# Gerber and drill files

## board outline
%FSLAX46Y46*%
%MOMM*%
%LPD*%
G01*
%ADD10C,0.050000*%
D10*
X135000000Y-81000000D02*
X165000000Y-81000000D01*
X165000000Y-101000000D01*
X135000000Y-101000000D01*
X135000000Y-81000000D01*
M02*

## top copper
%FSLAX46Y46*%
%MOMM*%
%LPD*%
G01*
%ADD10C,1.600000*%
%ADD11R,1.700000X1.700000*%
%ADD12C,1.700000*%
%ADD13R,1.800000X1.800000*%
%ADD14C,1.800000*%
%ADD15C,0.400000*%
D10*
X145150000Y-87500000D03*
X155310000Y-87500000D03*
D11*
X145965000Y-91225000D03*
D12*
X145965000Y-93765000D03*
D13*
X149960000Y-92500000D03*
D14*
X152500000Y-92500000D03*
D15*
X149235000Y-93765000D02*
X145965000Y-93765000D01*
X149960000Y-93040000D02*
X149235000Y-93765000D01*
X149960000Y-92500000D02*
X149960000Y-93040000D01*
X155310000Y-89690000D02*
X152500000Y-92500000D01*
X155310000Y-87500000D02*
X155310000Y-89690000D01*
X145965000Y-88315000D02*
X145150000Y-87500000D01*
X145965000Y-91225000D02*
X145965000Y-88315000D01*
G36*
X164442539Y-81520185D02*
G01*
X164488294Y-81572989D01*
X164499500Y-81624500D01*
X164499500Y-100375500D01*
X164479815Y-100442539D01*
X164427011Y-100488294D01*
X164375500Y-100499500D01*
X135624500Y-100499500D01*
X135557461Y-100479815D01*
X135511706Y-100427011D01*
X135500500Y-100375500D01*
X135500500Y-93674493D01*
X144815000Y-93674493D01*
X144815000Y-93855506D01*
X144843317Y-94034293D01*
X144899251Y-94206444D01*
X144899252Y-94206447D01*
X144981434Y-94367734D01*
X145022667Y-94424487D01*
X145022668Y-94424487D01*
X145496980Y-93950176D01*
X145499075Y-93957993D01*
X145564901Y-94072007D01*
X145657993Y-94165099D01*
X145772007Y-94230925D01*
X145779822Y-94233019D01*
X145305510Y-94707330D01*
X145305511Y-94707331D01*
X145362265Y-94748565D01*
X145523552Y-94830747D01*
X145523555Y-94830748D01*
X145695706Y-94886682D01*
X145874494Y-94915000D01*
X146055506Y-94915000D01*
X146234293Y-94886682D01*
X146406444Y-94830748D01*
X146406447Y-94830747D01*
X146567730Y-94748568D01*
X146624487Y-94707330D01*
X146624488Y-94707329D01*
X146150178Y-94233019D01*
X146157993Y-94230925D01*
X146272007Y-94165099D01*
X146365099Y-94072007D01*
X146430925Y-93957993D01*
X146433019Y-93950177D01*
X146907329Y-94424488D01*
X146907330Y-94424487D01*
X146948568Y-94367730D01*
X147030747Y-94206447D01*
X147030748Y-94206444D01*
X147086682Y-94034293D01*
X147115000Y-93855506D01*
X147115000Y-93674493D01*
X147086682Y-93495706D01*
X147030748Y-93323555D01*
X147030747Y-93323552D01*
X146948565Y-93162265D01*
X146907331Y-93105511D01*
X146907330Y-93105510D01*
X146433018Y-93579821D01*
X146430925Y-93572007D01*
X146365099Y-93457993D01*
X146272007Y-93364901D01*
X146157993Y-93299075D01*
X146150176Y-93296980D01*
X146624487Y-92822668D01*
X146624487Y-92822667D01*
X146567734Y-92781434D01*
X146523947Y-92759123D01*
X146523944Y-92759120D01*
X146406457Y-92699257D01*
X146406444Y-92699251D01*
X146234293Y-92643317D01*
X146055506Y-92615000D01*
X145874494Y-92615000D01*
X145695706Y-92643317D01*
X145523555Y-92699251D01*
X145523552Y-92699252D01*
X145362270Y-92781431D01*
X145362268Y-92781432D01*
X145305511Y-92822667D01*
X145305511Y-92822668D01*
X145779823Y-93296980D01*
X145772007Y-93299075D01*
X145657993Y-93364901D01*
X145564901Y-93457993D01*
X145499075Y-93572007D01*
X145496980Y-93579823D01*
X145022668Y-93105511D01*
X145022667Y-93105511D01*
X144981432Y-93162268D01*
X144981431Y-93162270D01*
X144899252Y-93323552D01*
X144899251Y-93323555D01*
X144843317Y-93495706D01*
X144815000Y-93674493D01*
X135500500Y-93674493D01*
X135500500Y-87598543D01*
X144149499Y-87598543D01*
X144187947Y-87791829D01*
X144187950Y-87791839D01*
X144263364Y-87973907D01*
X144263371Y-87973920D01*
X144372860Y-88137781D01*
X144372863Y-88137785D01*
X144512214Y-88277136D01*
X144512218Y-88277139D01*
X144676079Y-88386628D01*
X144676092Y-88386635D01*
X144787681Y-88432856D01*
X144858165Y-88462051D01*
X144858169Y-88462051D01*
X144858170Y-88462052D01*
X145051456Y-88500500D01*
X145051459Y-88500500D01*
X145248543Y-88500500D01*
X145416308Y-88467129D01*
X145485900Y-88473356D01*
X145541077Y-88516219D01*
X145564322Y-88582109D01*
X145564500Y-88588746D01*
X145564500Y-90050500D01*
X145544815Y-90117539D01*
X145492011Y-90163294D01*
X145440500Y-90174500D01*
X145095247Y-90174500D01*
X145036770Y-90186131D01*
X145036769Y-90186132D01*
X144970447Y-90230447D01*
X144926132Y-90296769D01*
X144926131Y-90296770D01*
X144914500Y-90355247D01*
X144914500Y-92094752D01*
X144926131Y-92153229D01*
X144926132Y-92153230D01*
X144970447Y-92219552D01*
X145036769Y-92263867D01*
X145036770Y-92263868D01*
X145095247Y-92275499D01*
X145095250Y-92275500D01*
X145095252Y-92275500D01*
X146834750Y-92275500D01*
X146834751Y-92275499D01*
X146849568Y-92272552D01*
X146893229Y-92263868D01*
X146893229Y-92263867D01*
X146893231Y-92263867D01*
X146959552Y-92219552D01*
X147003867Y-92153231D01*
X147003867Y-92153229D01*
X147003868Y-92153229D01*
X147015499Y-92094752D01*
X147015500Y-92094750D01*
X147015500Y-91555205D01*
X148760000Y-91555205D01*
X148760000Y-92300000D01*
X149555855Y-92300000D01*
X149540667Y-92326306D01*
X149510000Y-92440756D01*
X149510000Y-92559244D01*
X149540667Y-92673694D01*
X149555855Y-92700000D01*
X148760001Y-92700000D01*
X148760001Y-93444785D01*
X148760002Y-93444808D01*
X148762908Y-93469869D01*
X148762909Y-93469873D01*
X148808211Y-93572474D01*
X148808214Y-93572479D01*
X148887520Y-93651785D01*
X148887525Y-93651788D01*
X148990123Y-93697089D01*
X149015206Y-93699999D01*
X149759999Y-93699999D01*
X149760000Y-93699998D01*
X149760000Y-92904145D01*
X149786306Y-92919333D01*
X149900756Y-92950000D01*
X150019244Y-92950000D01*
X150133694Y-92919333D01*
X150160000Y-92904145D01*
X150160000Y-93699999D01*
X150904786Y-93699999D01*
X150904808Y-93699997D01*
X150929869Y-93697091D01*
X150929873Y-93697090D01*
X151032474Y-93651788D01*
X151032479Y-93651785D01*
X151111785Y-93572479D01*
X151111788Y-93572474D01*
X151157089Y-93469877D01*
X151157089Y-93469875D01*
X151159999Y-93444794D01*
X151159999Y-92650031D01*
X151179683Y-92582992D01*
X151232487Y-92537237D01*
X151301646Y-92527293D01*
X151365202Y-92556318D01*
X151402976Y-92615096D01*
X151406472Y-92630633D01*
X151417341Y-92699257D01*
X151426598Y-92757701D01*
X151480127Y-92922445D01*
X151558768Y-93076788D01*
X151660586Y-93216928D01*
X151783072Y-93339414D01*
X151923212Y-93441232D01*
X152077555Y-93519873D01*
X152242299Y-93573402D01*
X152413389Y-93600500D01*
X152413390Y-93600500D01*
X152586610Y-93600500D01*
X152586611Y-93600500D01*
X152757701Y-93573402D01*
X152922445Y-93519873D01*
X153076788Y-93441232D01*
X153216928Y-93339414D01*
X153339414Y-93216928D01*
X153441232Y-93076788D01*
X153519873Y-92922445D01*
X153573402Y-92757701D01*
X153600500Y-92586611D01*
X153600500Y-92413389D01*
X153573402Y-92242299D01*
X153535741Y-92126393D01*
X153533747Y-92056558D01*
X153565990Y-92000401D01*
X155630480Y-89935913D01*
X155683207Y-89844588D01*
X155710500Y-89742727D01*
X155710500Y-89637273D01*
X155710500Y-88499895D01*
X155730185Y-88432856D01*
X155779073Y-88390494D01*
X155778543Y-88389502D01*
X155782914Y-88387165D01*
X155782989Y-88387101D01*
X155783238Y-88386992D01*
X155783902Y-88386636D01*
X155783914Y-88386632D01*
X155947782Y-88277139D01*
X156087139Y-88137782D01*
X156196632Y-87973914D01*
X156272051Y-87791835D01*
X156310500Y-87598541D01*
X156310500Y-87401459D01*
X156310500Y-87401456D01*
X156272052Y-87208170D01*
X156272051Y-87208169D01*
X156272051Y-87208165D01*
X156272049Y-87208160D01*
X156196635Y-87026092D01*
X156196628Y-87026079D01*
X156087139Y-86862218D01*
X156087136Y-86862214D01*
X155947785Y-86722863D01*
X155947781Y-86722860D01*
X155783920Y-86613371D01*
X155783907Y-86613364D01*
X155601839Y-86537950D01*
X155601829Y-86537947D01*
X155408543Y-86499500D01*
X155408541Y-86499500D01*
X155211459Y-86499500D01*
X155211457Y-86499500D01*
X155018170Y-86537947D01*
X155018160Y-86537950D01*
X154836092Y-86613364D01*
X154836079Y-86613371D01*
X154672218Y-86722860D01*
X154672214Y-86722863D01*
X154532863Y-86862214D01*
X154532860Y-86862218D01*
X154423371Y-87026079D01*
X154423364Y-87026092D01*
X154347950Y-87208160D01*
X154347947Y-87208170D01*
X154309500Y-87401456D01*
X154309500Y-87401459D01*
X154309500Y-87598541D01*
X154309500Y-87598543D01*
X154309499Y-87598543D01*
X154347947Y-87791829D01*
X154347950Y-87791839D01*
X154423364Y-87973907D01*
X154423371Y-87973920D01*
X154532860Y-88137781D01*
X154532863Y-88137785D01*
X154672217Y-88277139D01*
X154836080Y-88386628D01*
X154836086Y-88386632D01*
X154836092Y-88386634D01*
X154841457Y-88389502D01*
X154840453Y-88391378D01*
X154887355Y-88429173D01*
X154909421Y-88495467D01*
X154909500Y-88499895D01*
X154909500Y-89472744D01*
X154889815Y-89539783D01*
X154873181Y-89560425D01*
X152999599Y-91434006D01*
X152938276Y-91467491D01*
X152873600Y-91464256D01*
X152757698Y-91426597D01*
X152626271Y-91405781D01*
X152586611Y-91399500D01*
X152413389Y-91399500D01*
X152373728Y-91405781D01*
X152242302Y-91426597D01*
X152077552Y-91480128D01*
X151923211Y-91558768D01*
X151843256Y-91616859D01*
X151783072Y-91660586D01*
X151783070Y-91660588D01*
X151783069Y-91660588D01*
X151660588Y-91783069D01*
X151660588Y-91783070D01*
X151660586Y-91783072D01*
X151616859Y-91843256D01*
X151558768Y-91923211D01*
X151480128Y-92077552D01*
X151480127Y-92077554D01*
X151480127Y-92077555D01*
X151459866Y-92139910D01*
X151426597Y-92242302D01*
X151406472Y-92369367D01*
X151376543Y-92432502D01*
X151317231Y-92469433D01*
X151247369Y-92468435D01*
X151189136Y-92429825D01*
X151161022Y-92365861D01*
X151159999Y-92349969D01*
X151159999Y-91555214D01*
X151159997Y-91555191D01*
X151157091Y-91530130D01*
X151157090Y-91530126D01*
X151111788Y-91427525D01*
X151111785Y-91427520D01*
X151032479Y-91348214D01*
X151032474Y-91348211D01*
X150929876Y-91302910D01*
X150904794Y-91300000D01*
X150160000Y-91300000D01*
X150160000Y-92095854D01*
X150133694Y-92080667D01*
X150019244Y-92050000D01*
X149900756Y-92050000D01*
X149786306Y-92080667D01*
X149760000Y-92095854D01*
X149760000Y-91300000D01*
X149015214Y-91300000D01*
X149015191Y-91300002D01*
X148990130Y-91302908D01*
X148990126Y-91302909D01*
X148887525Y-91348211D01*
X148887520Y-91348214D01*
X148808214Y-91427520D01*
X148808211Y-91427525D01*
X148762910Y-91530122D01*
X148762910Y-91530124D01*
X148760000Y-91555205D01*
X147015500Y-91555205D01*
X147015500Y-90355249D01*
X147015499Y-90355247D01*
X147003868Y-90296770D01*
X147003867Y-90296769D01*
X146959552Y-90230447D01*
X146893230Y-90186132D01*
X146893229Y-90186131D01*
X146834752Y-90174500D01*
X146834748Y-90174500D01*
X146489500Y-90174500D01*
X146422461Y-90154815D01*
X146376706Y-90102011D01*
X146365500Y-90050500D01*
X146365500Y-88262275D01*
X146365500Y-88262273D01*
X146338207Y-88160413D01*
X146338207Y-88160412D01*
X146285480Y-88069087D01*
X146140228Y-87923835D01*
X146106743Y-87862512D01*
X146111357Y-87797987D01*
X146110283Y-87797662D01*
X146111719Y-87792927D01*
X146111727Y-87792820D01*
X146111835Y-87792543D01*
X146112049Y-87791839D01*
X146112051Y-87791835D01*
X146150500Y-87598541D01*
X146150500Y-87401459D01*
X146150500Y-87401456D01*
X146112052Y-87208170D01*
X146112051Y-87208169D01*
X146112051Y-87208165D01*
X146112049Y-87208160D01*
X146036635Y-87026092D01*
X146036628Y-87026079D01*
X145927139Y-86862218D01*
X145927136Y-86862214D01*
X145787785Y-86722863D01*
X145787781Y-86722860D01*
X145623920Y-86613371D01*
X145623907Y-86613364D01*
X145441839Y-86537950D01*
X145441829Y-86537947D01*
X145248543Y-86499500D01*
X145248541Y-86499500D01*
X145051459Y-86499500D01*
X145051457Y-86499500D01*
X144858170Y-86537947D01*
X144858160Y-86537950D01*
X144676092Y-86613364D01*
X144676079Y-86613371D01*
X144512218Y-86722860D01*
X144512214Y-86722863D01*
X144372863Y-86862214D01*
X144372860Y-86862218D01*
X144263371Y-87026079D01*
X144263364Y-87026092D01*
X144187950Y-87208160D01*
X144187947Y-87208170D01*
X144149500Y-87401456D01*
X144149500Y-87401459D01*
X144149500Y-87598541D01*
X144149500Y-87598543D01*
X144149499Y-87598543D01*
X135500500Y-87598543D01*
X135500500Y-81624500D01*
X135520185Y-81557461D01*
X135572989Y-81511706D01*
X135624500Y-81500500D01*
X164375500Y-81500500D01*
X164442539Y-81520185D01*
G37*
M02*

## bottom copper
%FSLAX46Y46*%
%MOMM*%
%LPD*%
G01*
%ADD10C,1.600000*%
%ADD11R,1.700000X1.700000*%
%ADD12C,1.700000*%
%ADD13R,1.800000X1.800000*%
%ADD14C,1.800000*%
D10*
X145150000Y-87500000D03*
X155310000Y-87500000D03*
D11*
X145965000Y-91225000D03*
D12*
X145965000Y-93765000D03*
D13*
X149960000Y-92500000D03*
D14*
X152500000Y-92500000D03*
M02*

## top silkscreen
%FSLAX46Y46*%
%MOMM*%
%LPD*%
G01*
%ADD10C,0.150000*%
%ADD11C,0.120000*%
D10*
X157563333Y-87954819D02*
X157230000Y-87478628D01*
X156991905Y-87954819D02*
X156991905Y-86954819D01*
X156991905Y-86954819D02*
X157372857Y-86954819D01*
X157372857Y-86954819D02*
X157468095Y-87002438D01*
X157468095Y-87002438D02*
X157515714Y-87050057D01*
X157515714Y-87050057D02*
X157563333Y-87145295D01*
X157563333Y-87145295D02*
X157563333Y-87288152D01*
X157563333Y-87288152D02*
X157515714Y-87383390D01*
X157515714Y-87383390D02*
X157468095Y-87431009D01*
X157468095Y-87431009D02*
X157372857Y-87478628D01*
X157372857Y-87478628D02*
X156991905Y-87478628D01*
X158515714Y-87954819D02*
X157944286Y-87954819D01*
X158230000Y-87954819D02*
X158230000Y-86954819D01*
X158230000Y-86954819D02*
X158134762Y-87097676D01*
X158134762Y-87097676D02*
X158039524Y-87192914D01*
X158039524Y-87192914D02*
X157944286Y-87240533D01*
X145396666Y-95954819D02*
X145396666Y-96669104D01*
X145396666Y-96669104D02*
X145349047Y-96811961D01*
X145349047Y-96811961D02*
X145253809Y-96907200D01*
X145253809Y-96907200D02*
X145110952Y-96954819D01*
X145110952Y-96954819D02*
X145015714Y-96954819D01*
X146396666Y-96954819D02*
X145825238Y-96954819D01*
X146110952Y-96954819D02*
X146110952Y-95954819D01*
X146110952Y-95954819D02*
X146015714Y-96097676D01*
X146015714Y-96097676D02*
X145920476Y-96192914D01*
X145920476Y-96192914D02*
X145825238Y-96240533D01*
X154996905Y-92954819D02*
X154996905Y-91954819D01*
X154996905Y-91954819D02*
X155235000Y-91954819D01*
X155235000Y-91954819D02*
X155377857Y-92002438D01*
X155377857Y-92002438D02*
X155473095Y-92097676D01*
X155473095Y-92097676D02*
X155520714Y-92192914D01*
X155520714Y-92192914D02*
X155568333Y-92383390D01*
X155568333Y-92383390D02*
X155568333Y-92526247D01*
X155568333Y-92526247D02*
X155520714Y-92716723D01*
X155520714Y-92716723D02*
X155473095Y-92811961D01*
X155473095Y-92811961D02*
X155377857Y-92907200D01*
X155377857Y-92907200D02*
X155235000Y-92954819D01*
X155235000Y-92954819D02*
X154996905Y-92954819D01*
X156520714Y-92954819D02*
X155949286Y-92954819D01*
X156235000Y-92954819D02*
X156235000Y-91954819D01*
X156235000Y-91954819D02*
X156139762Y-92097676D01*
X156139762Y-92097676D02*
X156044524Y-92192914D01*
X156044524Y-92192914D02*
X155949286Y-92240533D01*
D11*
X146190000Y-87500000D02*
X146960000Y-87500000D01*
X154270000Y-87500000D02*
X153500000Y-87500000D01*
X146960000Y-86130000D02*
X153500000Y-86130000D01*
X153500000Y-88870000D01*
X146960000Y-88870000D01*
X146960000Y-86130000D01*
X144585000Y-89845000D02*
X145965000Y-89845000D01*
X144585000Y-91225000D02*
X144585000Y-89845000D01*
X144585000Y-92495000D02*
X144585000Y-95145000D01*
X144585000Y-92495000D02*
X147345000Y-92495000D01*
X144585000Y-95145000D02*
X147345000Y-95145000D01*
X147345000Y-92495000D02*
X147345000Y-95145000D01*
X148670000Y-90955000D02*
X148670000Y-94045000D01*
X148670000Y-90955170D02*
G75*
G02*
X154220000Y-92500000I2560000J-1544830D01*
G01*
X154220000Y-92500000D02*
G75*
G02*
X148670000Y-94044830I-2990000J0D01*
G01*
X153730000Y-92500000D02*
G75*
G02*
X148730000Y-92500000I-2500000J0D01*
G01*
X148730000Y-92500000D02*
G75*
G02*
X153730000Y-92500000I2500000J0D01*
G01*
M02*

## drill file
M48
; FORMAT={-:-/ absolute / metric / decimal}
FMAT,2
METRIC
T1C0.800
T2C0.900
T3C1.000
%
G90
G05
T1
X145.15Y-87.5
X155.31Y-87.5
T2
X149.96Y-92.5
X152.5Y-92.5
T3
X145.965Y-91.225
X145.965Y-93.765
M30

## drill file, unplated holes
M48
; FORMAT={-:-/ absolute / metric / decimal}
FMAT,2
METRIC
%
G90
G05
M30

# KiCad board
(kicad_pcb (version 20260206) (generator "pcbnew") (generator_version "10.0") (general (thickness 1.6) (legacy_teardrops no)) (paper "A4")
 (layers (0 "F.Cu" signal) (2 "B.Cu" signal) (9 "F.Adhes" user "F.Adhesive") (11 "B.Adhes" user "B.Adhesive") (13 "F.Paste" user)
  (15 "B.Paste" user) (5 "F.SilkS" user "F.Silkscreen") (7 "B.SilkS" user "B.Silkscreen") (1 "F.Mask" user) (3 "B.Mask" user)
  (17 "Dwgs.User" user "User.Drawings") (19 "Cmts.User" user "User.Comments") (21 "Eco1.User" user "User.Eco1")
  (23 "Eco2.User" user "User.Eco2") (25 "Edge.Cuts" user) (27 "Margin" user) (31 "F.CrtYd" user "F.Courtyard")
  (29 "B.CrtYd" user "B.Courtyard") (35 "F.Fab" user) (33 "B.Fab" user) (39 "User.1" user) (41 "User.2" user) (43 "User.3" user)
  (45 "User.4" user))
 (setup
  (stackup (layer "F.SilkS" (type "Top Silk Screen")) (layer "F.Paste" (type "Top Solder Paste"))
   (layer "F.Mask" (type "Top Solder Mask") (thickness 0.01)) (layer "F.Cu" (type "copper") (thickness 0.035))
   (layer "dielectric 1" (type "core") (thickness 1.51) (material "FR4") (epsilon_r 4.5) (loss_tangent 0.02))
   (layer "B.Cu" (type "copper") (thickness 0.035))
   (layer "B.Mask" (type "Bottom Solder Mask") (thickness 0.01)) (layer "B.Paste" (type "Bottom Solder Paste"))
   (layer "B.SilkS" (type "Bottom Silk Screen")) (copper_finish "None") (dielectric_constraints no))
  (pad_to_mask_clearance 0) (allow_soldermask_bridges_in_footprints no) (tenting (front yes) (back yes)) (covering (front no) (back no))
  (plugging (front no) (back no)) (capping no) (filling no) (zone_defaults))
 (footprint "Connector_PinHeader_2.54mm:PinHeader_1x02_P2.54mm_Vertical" (layer "F.Cu") (at 145.965 91.225)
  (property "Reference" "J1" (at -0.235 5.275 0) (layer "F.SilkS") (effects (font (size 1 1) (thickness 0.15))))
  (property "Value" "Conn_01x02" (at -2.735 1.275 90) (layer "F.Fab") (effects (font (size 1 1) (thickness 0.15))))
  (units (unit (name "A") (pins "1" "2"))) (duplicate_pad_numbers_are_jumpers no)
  (fp_line (start -1.38 -1.38) (end 0 -1.38) (stroke (width 0.12) (type solid)) (layer "F.SilkS"))
  (fp_line (start -1.38 0) (end -1.38 -1.38) (stroke (width 0.12) (type solid)) (layer "F.SilkS"))
  (fp_line (start -1.38 1.27) (end -1.38 3.92) (stroke (width 0.12) (type solid)) (layer "F.SilkS"))
  (fp_line (start -1.38 1.27) (end 1.38 1.27) (stroke (width 0.12) (type solid)) (layer "F.SilkS"))
  (fp_line (start -1.38 3.92) (end 1.38 3.92) (stroke (width 0.12) (type solid)) (layer "F.SilkS"))
  (fp_line (start 1.38 1.27) (end 1.38 3.92) (stroke (width 0.12) (type solid)) (layer "F.SilkS"))
  (pad "1" thru_hole rect (at 0 0) (size 1.7 1.7) (drill 1) (layers "*.Cu" "*.Mask") (remove_unused_layers no) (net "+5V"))
  (pad "2" thru_hole circle (at 0 2.54) (size 1.7 1.7) (drill 1) (layers "*.Cu" "*.Mask") (remove_unused_layers no) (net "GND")))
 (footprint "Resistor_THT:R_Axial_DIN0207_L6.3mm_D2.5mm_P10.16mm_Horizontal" (layer "F.Cu") (at 145.15 87.5)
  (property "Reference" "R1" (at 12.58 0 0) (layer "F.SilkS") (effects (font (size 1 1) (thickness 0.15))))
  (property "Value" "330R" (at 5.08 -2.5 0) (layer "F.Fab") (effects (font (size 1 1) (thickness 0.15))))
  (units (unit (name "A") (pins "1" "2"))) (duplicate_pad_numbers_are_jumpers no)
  (fp_line (start 1.04 0) (end 1.81 0) (stroke (width 0.12) (type solid)) (layer "F.SilkS"))
  (fp_line (start 9.12 0) (end 8.35 0) (stroke (width 0.12) (type solid)) (layer "F.SilkS"))
  (fp_rect (start 1.81 -1.37) (end 8.35 1.37) (stroke (width 0.12) (type solid)) (fill no) (layer "F.SilkS"))
  (pad "1" thru_hole circle (at 0 0) (size 1.6 1.6) (drill 0.8) (layers "*.Cu" "*.Mask") (remove_unused_layers no) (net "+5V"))
  (pad "2" thru_hole circle (at 10.16 0) (size 1.6 1.6) (drill 0.8) (layers "*.Cu" "*.Mask") (remove_unused_layers no) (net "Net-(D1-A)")))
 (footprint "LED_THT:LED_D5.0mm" (layer "F.Cu") (at 149.96 92.5)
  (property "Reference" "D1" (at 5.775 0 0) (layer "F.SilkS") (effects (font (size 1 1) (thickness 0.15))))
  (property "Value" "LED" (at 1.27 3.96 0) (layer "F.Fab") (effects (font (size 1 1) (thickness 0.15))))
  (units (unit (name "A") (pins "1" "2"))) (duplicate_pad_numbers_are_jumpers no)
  (fp_line (start -1.29 -1.545) (end -1.29 1.545) (stroke (width 0.12) (type solid)) (layer "F.SilkS"))
  (fp_arc (start -1.29 -1.54483) (mid 2.071779 -2.880495) (end 4.26 0) (stroke (width 0.12) (type solid)) (layer "F.SilkS"))
  (fp_arc (start 4.26 0) (mid 2.071779 2.880495) (end -1.29 1.54483) (stroke (width 0.12) (type solid)) (layer "F.SilkS"))
  (fp_circle (center 1.27 0) (end 3.77 0) (stroke (width 0.12) (type solid)) (fill no) (layer "F.SilkS"))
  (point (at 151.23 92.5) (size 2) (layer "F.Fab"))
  (pad "1" thru_hole rect (at 0 0) (size 1.8 1.8) (drill 0.9) (layers "*.Cu" "*.Mask") (remove_unused_layers no) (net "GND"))
  (pad "2" thru_hole circle (at 2.54 0) (size 1.8 1.8) (drill 0.9) (layers "*.Cu" "*.Mask") (remove_unused_layers no) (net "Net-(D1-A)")))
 (gr_rect (start 135 81) (end 165 101) (stroke (width 0.05) (type default)) (fill no) (layer "Edge.Cuts"))
 (segment (start 155.31 87.5) (end 155.31 89.69) (width 0.4) (layer "F.Cu") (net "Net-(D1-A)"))
 (segment (start 155.31 89.69) (end 152.5 92.5) (width 0.4) (layer "F.Cu") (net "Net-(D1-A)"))
 (segment (start 149.235 93.765) (end 145.965 93.765) (width 0.4) (layer "F.Cu") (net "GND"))
 (segment (start 149.96 93.04) (end 149.235 93.765) (width 0.4) (layer "F.Cu") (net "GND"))
 (segment (start 149.96 92.5) (end 149.96 93.04) (width 0.4) (layer "F.Cu") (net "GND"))
 (segment (start 145.965 88.315) (end 145.15 87.5) (width 0.4) (layer "F.Cu") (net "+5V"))
 (segment (start 145.965 91.225) (end 145.965 88.315) (width 0.4) (layer "F.Cu") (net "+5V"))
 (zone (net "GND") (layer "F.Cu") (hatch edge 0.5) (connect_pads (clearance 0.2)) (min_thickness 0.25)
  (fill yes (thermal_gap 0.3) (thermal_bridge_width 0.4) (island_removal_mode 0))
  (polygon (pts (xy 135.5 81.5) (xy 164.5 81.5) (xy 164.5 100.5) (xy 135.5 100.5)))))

